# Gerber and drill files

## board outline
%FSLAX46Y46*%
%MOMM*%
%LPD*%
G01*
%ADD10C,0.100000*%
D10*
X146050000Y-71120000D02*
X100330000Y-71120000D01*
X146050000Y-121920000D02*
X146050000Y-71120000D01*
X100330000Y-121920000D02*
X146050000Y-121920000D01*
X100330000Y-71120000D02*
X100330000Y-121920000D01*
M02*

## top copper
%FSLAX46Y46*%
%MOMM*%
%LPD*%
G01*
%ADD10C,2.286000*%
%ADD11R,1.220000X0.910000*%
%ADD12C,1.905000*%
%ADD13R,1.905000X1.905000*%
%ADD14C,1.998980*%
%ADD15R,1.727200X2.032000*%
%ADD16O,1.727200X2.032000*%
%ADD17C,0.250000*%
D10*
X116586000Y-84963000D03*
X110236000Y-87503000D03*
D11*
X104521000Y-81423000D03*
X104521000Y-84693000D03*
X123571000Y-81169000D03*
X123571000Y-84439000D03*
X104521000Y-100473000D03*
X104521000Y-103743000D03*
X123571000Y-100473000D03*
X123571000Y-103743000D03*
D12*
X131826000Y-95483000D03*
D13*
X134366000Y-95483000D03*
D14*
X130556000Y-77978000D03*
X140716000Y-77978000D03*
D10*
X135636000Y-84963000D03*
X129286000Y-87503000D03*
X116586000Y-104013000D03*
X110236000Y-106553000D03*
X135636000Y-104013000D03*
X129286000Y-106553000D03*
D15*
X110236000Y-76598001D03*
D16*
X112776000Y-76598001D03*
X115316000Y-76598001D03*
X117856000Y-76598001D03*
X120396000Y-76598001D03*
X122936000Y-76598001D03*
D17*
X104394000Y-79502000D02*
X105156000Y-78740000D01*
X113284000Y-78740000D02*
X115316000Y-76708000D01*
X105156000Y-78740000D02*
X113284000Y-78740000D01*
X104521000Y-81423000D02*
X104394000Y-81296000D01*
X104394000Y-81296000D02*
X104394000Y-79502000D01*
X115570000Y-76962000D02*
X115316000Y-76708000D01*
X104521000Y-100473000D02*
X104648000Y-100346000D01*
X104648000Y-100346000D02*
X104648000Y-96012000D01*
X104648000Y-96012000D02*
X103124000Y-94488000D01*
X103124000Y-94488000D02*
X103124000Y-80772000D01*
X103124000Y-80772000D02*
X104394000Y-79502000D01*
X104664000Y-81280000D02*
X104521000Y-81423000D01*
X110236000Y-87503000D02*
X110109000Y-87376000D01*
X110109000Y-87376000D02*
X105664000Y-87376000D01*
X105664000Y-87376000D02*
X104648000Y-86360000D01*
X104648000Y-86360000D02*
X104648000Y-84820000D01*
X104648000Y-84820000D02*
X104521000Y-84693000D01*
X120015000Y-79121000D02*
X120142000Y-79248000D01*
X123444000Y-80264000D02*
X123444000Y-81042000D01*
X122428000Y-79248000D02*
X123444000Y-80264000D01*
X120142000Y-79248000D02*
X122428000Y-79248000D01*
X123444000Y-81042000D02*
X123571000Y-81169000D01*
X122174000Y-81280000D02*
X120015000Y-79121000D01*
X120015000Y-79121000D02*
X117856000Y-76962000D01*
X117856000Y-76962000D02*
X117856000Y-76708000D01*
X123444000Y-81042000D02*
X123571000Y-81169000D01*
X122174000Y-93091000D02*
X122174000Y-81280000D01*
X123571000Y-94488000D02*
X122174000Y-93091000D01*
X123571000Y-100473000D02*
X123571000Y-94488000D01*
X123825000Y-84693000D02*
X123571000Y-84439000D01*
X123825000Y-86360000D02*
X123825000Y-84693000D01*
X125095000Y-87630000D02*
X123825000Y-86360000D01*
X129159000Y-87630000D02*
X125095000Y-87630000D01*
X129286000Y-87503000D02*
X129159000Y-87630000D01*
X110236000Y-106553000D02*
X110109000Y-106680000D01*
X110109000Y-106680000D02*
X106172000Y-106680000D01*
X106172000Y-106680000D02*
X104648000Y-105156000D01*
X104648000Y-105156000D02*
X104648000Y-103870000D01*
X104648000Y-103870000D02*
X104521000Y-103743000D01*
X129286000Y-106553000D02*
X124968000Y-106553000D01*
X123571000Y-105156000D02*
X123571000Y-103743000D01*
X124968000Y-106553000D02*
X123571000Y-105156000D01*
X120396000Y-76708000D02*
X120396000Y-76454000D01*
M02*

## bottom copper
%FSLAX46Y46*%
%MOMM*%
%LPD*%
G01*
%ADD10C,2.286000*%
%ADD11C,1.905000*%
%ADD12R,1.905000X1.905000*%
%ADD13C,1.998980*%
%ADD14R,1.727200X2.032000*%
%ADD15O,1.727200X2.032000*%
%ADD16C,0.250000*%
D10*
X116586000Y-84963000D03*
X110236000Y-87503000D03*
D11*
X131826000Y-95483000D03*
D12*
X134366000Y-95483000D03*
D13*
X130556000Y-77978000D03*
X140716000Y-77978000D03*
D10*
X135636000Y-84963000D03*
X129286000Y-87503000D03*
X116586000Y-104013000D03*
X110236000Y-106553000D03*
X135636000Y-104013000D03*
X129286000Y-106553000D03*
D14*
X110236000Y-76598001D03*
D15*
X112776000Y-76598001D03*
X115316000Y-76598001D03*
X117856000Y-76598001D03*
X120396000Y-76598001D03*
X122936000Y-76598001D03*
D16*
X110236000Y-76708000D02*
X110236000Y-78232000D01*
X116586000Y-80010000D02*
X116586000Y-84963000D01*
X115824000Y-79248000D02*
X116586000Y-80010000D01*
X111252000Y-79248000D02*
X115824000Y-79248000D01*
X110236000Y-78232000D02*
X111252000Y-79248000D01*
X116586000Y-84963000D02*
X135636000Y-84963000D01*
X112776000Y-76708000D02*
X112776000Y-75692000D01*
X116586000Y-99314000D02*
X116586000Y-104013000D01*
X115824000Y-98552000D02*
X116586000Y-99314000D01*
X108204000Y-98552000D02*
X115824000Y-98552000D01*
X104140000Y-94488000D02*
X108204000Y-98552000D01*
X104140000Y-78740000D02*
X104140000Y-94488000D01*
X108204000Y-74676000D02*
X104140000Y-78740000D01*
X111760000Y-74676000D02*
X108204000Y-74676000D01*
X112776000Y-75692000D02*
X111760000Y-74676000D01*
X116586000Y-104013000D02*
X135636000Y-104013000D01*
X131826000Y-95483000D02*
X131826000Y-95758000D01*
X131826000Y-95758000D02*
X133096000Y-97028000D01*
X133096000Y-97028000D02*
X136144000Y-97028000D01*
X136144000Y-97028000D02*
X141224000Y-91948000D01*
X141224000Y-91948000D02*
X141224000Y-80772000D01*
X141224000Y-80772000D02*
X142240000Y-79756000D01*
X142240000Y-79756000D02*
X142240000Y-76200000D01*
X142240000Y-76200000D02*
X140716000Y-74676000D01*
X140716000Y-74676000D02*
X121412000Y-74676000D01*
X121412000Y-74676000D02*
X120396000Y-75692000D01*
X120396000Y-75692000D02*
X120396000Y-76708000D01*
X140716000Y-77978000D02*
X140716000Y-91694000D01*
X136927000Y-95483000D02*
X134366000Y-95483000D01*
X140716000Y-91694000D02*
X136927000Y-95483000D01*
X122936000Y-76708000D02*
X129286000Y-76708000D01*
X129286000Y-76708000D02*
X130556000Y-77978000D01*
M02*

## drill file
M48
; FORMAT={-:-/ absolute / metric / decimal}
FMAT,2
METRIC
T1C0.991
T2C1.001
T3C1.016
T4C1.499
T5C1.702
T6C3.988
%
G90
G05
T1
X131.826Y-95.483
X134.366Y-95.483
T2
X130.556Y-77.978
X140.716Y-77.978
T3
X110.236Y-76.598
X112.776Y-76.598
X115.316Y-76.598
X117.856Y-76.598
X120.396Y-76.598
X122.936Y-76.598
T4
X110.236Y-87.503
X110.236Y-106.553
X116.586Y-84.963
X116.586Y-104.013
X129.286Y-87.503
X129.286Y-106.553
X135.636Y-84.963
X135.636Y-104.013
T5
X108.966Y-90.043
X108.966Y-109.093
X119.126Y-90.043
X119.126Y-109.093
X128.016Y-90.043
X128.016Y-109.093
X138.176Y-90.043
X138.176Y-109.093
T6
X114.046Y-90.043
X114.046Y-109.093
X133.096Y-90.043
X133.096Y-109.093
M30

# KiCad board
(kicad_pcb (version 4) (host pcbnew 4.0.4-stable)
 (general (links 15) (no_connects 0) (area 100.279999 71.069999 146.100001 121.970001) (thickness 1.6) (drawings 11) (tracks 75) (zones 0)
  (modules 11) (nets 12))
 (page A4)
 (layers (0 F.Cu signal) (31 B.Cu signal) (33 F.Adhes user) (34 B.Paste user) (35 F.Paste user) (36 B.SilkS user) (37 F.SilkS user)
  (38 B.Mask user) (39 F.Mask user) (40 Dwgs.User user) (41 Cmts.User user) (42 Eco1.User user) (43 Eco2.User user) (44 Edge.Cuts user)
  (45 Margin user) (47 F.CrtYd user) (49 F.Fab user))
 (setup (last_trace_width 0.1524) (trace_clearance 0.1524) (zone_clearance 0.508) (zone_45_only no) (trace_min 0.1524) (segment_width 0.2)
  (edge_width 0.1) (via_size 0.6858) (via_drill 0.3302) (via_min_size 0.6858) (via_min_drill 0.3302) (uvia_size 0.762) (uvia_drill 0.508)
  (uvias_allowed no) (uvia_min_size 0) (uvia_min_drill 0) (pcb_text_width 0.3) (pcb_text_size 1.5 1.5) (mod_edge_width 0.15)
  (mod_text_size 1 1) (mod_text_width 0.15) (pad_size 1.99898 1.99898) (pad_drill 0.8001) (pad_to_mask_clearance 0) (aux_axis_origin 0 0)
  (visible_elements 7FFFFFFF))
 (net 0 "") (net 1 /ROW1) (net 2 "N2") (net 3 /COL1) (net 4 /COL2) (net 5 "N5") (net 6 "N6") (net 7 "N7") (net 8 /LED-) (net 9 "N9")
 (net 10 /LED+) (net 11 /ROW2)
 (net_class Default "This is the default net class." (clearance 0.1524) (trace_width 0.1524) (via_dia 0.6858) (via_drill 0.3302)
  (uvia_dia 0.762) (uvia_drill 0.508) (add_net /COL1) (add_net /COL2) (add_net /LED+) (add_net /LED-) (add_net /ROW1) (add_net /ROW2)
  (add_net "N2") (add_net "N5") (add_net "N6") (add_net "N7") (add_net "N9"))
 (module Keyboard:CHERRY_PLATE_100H (layer F.Cu) (at 114.046 90.043)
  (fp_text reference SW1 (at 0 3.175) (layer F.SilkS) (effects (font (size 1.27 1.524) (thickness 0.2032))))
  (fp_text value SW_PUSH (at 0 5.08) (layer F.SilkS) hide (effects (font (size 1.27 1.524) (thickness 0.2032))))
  (pad 1 thru_hole circle (at 2.54 -5.08) (size 2.286 2.286) (drill 1.4986) (layers *.Cu *.SilkS *.Mask) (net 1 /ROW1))
  (pad 2 thru_hole circle (at -3.81 -2.54) (size 2.286 2.286) (drill 1.4986) (layers *.Cu *.SilkS *.Mask) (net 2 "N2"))
  (pad HOLE np_thru_hole circle (at 0 0) (size 3.9878 3.9878) (drill 3.9878) (layers *.Cu))
  (pad HOLE np_thru_hole circle (at -5.08 0) (size 1.7018 1.7018) (drill 1.7018) (layers *.Cu))
  (pad HOLE np_thru_hole circle (at 5.08 0) (size 1.7018 1.7018) (drill 1.7018) (layers *.Cu)))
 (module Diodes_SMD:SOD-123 (layer F.Cu) (at 104.521 83.058 270)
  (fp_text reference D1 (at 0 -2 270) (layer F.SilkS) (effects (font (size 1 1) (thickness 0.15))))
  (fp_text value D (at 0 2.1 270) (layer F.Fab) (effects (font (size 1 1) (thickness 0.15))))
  (pad 1 smd rect (at -1.635 0 270) (size 0.91 1.22) (layers F.Cu F.Paste F.Mask) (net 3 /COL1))
  (pad 2 smd rect (at 1.635 0 270) (size 0.91 1.22) (layers F.Cu F.Paste F.Mask) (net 2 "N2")))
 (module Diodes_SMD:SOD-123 (layer F.Cu) (at 123.571 82.804 270)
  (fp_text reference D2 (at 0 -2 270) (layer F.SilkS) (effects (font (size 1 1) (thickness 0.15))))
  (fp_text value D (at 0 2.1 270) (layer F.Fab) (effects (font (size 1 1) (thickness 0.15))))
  (pad 1 smd rect (at -1.635 0 270) (size 0.91 1.22) (layers F.Cu F.Paste F.Mask) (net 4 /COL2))
  (pad 2 smd rect (at 1.635 0 270) (size 0.91 1.22) (layers F.Cu F.Paste F.Mask) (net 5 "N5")))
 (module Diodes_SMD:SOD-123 (layer F.Cu) (at 104.521 102.108 270)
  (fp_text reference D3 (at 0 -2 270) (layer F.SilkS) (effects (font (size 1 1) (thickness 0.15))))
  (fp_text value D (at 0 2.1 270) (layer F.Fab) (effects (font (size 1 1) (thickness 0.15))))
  (pad 1 smd rect (at -1.635 0 270) (size 0.91 1.22) (layers F.Cu F.Paste F.Mask) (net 3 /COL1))
  (pad 2 smd rect (at 1.635 0 270) (size 0.91 1.22) (layers F.Cu F.Paste F.Mask) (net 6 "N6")))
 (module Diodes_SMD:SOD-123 (layer F.Cu) (at 123.571 102.108 270)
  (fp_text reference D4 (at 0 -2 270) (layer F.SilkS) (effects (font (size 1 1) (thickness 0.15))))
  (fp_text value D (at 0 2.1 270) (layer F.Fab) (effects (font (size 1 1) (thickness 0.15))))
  (pad 1 smd rect (at -1.635 0 270) (size 0.91 1.22) (layers F.Cu F.Paste F.Mask) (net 4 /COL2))
  (pad 2 smd rect (at 1.635 0 270) (size 0.91 1.22) (layers F.Cu F.Paste F.Mask) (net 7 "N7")))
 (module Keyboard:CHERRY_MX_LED (layer F.Cu) (at 133.096 90.403)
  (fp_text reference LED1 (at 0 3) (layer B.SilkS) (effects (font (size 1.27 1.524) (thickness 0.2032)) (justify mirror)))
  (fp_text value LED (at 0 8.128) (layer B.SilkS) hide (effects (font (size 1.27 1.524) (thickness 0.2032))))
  (pad 1 thru_hole circle (at -1.27 5.08) (size 1.905 1.905) (drill 0.9906) (layers *.Cu *.SilkS *.Mask) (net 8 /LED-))
  (pad 2 thru_hole rect (at 1.27 5.08) (size 1.905 1.905) (drill 0.9906) (layers *.Cu *.SilkS *.Mask) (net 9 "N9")))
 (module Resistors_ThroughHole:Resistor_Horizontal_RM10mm (layer F.Cu) (at 130.556 77.978)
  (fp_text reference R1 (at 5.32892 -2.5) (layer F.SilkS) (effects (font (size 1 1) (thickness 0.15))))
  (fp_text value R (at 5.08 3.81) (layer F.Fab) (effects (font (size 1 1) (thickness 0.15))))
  (pad 1 thru_hole circle (at 0 0) (size 1.99898 1.99898) (drill 1.00076) (layers *.Cu *.SilkS *.Mask) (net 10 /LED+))
  (pad 2 thru_hole circle (at 10.16 0) (size 1.99898 1.99898) (drill 1.00076) (layers *.Cu *.SilkS *.Mask) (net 9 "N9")))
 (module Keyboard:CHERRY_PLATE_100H (layer F.Cu) (at 133.096 90.043)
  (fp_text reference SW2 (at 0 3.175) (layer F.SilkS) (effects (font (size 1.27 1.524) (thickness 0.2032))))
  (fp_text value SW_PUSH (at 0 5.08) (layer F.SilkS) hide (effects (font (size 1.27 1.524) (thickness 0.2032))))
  (pad 1 thru_hole circle (at 2.54 -5.08) (size 2.286 2.286) (drill 1.4986) (layers *.Cu *.SilkS *.Mask) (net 1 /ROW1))
  (pad 2 thru_hole circle (at -3.81 -2.54) (size 2.286 2.286) (drill 1.4986) (layers *.Cu *.SilkS *.Mask) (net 5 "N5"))
  (pad HOLE np_thru_hole circle (at 0 0) (size 3.9878 3.9878) (drill 3.9878) (layers *.Cu))
  (pad HOLE np_thru_hole circle (at -5.08 0) (size 1.7018 1.7018) (drill 1.7018) (layers *.Cu))
  (pad HOLE np_thru_hole circle (at 5.08 0) (size 1.7018 1.7018) (drill 1.7018) (layers *.Cu)))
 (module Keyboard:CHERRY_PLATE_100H (layer F.Cu) (at 114.046 109.093)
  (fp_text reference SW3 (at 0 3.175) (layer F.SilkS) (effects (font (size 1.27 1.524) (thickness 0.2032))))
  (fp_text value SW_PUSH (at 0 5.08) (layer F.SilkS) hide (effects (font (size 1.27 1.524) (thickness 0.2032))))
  (pad 1 thru_hole circle (at 2.54 -5.08) (size 2.286 2.286) (drill 1.4986) (layers *.Cu *.SilkS *.Mask) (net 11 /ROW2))
  (pad 2 thru_hole circle (at -3.81 -2.54) (size 2.286 2.286) (drill 1.4986) (layers *.Cu *.SilkS *.Mask) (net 6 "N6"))
  (pad HOLE np_thru_hole circle (at 0 0) (size 3.9878 3.9878) (drill 3.9878) (layers *.Cu))
  (pad HOLE np_thru_hole circle (at -5.08 0) (size 1.7018 1.7018) (drill 1.7018) (layers *.Cu))
  (pad HOLE np_thru_hole circle (at 5.08 0) (size 1.7018 1.7018) (drill 1.7018) (layers *.Cu)))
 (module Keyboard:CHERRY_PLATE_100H (layer F.Cu) (at 133.096 109.093)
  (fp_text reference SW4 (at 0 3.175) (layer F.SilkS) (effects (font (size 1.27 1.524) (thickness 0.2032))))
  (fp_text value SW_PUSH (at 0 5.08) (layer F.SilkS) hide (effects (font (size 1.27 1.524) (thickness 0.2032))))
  (pad 1 thru_hole circle (at 2.54 -5.08) (size 2.286 2.286) (drill 1.4986) (layers *.Cu *.SilkS *.Mask) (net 11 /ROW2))
  (pad 2 thru_hole circle (at -3.81 -2.54) (size 2.286 2.286) (drill 1.4986) (layers *.Cu *.SilkS *.Mask) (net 7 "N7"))
  (pad HOLE np_thru_hole circle (at 0 0) (size 3.9878 3.9878) (drill 3.9878) (layers *.Cu))
  (pad HOLE np_thru_hole circle (at -5.08 0) (size 1.7018 1.7018) (drill 1.7018) (layers *.Cu))
  (pad HOLE np_thru_hole circle (at 5.08 0) (size 1.7018 1.7018) (drill 1.7018) (layers *.Cu)))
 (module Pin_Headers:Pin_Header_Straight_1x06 (layer F.Cu) (at 110.236 76.598001 90)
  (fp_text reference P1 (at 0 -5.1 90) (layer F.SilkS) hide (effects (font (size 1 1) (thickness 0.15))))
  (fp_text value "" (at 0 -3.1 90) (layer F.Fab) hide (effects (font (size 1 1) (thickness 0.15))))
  (pad 1 thru_hole rect (at 0 0 90) (size 2.032 1.7272) (drill 1.016) (layers *.Cu *.Mask F.SilkS) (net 1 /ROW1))
  (pad 2 thru_hole oval (at 0 2.54 90) (size 2.032 1.7272) (drill 1.016) (layers *.Cu *.Mask F.SilkS) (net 11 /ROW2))
  (pad 3 thru_hole oval (at 0 5.08 90) (size 2.032 1.7272) (drill 1.016) (layers *.Cu *.Mask F.SilkS) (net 3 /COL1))
  (pad 4 thru_hole oval (at 0 7.62 90) (size 2.032 1.7272) (drill 1.016) (layers *.Cu *.Mask F.SilkS) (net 4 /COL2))
  (pad 5 thru_hole oval (at 0 10.16 90) (size 2.032 1.7272) (drill 1.016) (layers *.Cu *.Mask F.SilkS) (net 8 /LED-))
  (pad 6 thru_hole oval (at 0 12.7 90) (size 2.032 1.7272) (drill 1.016) (layers *.Cu *.Mask F.SilkS) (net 10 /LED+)))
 (gr_line (start 146.05 71.12) (end 100.33 71.12) (angle 90) (layer Edge.Cuts) (width 0.1))
 (gr_line (start 146.05 121.92) (end 146.05 71.12) (angle 90) (layer Edge.Cuts) (width 0.1))
 (gr_line (start 100.33 121.92) (end 146.05 121.92) (angle 90) (layer Edge.Cuts) (width 0.1))
 (gr_line (start 100.33 71.12) (end 100.33 121.92) (angle 90) (layer Edge.Cuts) (width 0.1))
 (segment (start 104.394 79.502) (end 105.156 78.74) (width 0.25) (layer F.Cu) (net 3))
 (segment (start 113.284 78.74) (end 115.316 76.708) (width 0.25) (layer F.Cu) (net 3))
 (segment (start 105.156 78.74) (end 113.284 78.74) (width 0.25) (layer F.Cu) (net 3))
 (segment (start 104.521 81.423) (end 104.394 81.296) (width 0.25) (layer F.Cu) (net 3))
 (segment (start 104.394 81.296) (end 104.394 79.502) (width 0.25) (layer F.Cu) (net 3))
 (segment (start 115.57 76.962) (end 115.316 76.708) (width 0.25) (layer F.Cu) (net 3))
 (segment (start 104.521 100.473) (end 104.648 100.346) (width 0.25) (layer F.Cu) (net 3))
 (segment (start 104.648 100.346) (end 104.648 96.012) (width 0.25) (layer F.Cu) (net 3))
 (segment (start 104.648 96.012) (end 103.124 94.488) (width 0.25) (layer F.Cu) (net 3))
 (segment (start 103.124 94.488) (end 103.124 80.772) (width 0.25) (layer F.Cu) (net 3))
 (segment (start 103.124 80.772) (end 104.394 79.502) (width 0.25) (layer F.Cu) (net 3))
 (segment (start 104.664 81.28) (end 104.521 81.423) (width 0.25) (layer F.Cu) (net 3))
 (segment (start 110.236 87.503) (end 110.109 87.376) (width 0.25) (layer F.Cu) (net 2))
 (segment (start 110.109 87.376) (end 105.664 87.376) (width 0.25) (layer F.Cu) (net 2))
 (segment (start 105.664 87.376) (end 104.648 86.36) (width 0.25) (layer F.Cu) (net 2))
 (segment (start 104.648 86.36) (end 104.648 84.82) (width 0.25) (layer F.Cu) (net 2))
 (segment (start 104.648 84.82) (end 104.521 84.693) (width 0.25) (layer F.Cu) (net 2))
 (segment (start 120.015 79.121) (end 120.142 79.248) (width 0.25) (layer F.Cu) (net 4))
 (segment (start 123.444 80.264) (end 123.444 81.042) (width 0.25) (layer F.Cu) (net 4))
 (segment (start 122.428 79.248) (end 123.444 80.264) (width 0.25) (layer F.Cu) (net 4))
 (segment (start 120.142 79.248) (end 122.428 79.248) (width 0.25) (layer F.Cu) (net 4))
 (segment (start 123.444 81.042) (end 123.571 81.169) (width 0.25) (layer F.Cu) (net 4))
 (segment (start 122.174 81.28) (end 120.015 79.121) (width 0.25) (layer F.Cu) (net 4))
 (segment (start 120.015 79.121) (end 117.856 76.962) (width 0.25) (layer F.Cu) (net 4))
 (segment (start 117.856 76.962) (end 117.856 76.708) (width 0.25) (layer F.Cu) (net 4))
 (segment (start 123.444 81.042) (end 123.571 81.169) (width 0.25) (layer F.Cu) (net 4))
 (segment (start 122.174 93.091) (end 122.174 81.28) (width 0.25) (layer F.Cu) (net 4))
 (segment (start 123.571 94.488) (end 122.174 93.091) (width 0.25) (layer F.Cu) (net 4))
 (segment (start 123.571 100.473) (end 123.571 94.488) (width 0.25) (layer F.Cu) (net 4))
 (segment (start 123.825 84.693) (end 123.571 84.439) (width 0.25) (layer F.Cu) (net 5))
 (segment (start 123.825 86.36) (end 123.825 84.693) (width 0.25) (layer F.Cu) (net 5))
 (segment (start 125.095 87.63) (end 123.825 86.36) (width 0.25) (layer F.Cu) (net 5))
 (segment (start 129.159 87.63) (end 125.095 87.63) (width 0.25) (layer F.Cu) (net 5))
 (segment (start 129.286 87.503) (end 129.159 87.63) (width 0.25) (layer F.Cu) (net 5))
 (segment (start 110.236 106.553) (end 110.109 106.68) (width 0.25) (layer F.Cu) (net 6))
 (segment (start 110.109 106.68) (end 106.172 106.68) (width 0.25) (layer F.Cu) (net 6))
 (segment (start 106.172 106.68) (end 104.648 105.156) (width 0.25) (layer F.Cu) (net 6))
 (segment (start 104.648 105.156) (end 104.648 103.87) (width 0.25) (layer F.Cu) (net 6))
 (segment (start 104.648 103.87) (end 104.521 103.743) (width 0.25) (layer F.Cu) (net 6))
 (segment (start 129.286 106.553) (end 124.968 106.553) (width 0.25) (layer F.Cu) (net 7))
 (segment (start 123.571 105.156) (end 123.571 103.743) (width 0.25) (layer F.Cu) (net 7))
 (segment (start 124.968 106.553) (end 123.571 105.156) (width 0.25) (layer F.Cu) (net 7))
 (segment (start 110.236 76.708) (end 110.236 78.232) (width 0.25) (layer B.Cu) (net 1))
 (segment (start 116.586 80.01) (end 116.586 84.963) (width 0.25) (layer B.Cu) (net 1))
 (segment (start 115.824 79.248) (end 116.586 80.01) (width 0.25) (layer B.Cu) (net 1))
 (segment (start 111.252 79.248) (end 115.824 79.248) (width 0.25) (layer B.Cu) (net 1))
 (segment (start 110.236 78.232) (end 111.252 79.248) (width 0.25) (layer B.Cu) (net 1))
 (segment (start 116.586 84.963) (end 135.636 84.963) (width 0.25) (layer B.Cu) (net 1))
 (segment (start 112.776 76.708) (end 112.776 75.692) (width 0.25) (layer B.Cu) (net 11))
 (segment (start 116.586 99.314) (end 116.586 104.013) (width 0.25) (layer B.Cu) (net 11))
 (segment (start 115.824 98.552) (end 116.586 99.314) (width 0.25) (layer B.Cu) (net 11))
 (segment (start 108.204 98.552) (end 115.824 98.552) (width 0.25) (layer B.Cu) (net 11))
 (segment (start 104.14 94.488) (end 108.204 98.552) (width 0.25) (layer B.Cu) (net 11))
 (segment (start 104.14 78.74) (end 104.14 94.488) (width 0.25) (layer B.Cu) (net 11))
 (segment (start 108.204 74.676) (end 104.14 78.74) (width 0.25) (layer B.Cu) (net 11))
 (segment (start 111.76 74.676) (end 108.204 74.676) (width 0.25) (layer B.Cu) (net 11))
 (segment (start 112.776 75.692) (end 111.76 74.676) (width 0.25) (layer B.Cu) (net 11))
 (segment (start 116.586 104.013) (end 135.636 104.013) (width 0.25) (layer B.Cu) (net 11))
 (segment (start 120.396 76.708) (end 120.396 76.454) (width 0.25) (layer F.Cu) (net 8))
 (segment (start 131.826 95.483) (end 131.826 95.758) (width 0.25) (layer B.Cu) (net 8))
 (segment (start 131.826 95.758) (end 133.096 97.028) (width 0.25) (layer B.Cu) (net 8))
 (segment (start 133.096 97.028) (end 136.144 97.028) (width 0.25) (layer B.Cu) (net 8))
 (segment (start 136.144 97.028) (end 141.224 91.948) (width 0.25) (layer B.Cu) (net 8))
 (segment (start 141.224 91.948) (end 141.224 80.772) (width 0.25) (layer B.Cu) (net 8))
 (segment (start 141.224 80.772) (end 142.24 79.756) (width 0.25) (layer B.Cu) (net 8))
 (segment (start 142.24 79.756) (end 142.24 76.2) (width 0.25) (layer B.Cu) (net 8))
 (segment (start 142.24 76.2) (end 140.716 74.676) (width 0.25) (layer B.Cu) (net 8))
 (segment (start 140.716 74.676) (end 121.412 74.676) (width 0.25) (layer B.Cu) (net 8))
 (segment (start 121.412 74.676) (end 120.396 75.692) (width 0.25) (layer B.Cu) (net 8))
 (segment (start 120.396 75.692) (end 120.396 76.708) (width 0.25) (layer B.Cu) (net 8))
 (segment (start 140.716 77.978) (end 140.716 91.694) (width 0.25) (layer B.Cu) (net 9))
 (segment (start 136.927 95.483) (end 134.366 95.483) (width 0.25) (layer B.Cu) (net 9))
 (segment (start 140.716 91.694) (end 136.927 95.483) (width 0.25) (layer B.Cu) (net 9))
 (segment (start 122.936 76.708) (end 129.286 76.708) (width 0.25) (layer B.Cu) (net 10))
 (segment (start 129.286 76.708) (end 130.556 77.978) (width 0.25) (layer B.Cu) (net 10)))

